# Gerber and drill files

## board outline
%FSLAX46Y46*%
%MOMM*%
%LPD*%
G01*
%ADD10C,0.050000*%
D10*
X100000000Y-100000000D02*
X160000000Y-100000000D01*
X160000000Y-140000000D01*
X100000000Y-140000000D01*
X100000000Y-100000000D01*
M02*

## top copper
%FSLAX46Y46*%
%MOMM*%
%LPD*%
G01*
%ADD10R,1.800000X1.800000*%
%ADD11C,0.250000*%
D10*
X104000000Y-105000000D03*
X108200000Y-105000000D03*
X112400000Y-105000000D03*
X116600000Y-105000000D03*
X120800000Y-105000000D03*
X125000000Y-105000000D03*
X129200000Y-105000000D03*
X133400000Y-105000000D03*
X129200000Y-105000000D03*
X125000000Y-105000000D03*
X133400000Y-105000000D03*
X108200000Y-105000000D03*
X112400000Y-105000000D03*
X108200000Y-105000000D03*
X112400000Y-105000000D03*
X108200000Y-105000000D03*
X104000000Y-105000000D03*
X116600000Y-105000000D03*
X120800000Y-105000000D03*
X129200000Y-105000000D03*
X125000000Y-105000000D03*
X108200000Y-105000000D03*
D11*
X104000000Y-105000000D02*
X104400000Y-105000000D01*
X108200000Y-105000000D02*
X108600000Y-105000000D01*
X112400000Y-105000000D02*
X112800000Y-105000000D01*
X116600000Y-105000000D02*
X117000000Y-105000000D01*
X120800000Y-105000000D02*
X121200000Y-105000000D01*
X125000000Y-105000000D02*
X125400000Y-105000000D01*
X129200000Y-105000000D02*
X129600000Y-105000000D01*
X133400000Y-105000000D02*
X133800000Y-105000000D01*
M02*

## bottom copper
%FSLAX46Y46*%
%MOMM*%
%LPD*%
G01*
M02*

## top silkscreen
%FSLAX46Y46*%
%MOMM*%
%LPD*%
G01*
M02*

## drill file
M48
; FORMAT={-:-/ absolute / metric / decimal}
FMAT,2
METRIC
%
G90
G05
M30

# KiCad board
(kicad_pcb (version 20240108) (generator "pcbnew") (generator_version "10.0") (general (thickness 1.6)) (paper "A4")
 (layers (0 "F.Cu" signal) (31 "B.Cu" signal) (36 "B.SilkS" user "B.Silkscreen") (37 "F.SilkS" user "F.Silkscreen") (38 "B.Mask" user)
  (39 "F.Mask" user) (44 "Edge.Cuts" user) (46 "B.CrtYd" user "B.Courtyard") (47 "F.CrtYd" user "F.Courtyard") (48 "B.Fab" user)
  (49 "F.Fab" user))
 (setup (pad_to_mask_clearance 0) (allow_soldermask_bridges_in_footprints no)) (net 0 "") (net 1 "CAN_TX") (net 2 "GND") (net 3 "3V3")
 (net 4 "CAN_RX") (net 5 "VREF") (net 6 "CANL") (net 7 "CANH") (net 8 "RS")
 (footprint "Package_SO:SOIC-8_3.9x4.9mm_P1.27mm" (layer "F.Cu") (at 100 100)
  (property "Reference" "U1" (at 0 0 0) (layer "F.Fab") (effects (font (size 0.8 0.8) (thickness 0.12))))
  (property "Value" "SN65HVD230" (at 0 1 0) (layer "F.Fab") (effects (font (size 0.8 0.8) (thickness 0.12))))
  (pad "1" smd rect (at 4.000 5.000) (size 1.8 1.8) (layers "F.Cu" "F.Paste" "F.Mask") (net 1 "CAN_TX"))
  (pad "2" smd rect (at 8.200 5.000) (size 1.8 1.8) (layers "F.Cu" "F.Paste" "F.Mask") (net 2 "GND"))
  (pad "3" smd rect (at 12.400 5.000) (size 1.8 1.8) (layers "F.Cu" "F.Paste" "F.Mask") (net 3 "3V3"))
  (pad "4" smd rect (at 16.600 5.000) (size 1.8 1.8) (layers "F.Cu" "F.Paste" "F.Mask") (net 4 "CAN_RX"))
  (pad "5" smd rect (at 20.800 5.000) (size 1.8 1.8) (layers "F.Cu" "F.Paste" "F.Mask") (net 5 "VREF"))
  (pad "6" smd rect (at 25.000 5.000) (size 1.8 1.8) (layers "F.Cu" "F.Paste" "F.Mask") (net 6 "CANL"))
  (pad "7" smd rect (at 29.200 5.000) (size 1.8 1.8) (layers "F.Cu" "F.Paste" "F.Mask") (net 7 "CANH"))
  (pad "8" smd rect (at 33.400 5.000) (size 1.8 1.8) (layers "F.Cu" "F.Paste" "F.Mask") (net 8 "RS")))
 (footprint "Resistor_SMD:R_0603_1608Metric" (layer "F.Cu") (at 100 100)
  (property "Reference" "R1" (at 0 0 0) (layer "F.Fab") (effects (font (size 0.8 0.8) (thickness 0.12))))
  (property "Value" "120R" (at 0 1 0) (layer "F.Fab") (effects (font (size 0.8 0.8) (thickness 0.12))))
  (pad "1" smd rect (at 29.200 5.000) (size 1.8 1.8) (layers "F.Cu" "F.Paste" "F.Mask") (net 7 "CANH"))
  (pad "2" smd rect (at 25.000 5.000) (size 1.8 1.8) (layers "F.Cu" "F.Paste" "F.Mask") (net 6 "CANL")))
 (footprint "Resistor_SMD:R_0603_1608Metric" (layer "F.Cu") (at 100 100)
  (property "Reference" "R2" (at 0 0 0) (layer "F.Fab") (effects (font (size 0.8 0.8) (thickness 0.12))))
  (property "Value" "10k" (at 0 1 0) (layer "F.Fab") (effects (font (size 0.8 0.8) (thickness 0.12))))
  (pad "1" smd rect (at 33.400 5.000) (size 1.8 1.8) (layers "F.Cu" "F.Paste" "F.Mask") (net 8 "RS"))
  (pad "2" smd rect (at 8.200 5.000) (size 1.8 1.8) (layers "F.Cu" "F.Paste" "F.Mask") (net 2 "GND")))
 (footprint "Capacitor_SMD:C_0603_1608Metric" (layer "F.Cu") (at 100 100)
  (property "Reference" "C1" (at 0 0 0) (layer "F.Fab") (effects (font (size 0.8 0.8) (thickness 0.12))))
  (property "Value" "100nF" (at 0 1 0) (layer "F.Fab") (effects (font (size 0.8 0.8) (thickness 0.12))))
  (pad "1" smd rect (at 12.400 5.000) (size 1.8 1.8) (layers "F.Cu" "F.Paste" "F.Mask") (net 3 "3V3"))
  (pad "2" smd rect (at 8.200 5.000) (size 1.8 1.8) (layers "F.Cu" "F.Paste" "F.Mask") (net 2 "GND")))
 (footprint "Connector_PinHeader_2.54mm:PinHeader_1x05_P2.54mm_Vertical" (layer "F.Cu") (at 100 100)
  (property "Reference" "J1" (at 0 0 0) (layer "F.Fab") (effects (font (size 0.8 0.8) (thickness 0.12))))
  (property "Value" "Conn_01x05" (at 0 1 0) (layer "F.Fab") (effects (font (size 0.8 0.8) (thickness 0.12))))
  (pad "1" smd rect (at 12.400 5.000) (size 1.8 1.8) (layers "F.Cu" "F.Paste" "F.Mask") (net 3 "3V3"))
  (pad "2" smd rect (at 8.200 5.000) (size 1.8 1.8) (layers "F.Cu" "F.Paste" "F.Mask") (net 2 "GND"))
  (pad "3" smd rect (at 4.000 5.000) (size 1.8 1.8) (layers "F.Cu" "F.Paste" "F.Mask") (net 1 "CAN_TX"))
  (pad "4" smd rect (at 16.600 5.000) (size 1.8 1.8) (layers "F.Cu" "F.Paste" "F.Mask") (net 4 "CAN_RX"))
  (pad "5" smd rect (at 20.800 5.000) (size 1.8 1.8) (layers "F.Cu" "F.Paste" "F.Mask") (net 5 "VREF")))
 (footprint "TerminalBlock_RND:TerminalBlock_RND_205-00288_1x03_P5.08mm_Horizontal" (layer "F.Cu") (at 100 100)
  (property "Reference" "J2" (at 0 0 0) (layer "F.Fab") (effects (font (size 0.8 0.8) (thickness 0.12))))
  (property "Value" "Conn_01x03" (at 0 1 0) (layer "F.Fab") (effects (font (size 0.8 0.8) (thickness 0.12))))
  (pad "1" smd rect (at 29.200 5.000) (size 1.8 1.8) (layers "F.Cu" "F.Paste" "F.Mask") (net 7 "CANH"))
  (pad "2" smd rect (at 25.000 5.000) (size 1.8 1.8) (layers "F.Cu" "F.Paste" "F.Mask") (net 6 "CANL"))
  (pad "3" smd rect (at 8.200 5.000) (size 1.8 1.8) (layers "F.Cu" "F.Paste" "F.Mask") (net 2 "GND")))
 (gr_rect (start 100 100) (end 160 140) (stroke (width 0.05) (type default)) (fill none) (layer "Edge.Cuts"))
 (segment (start 104.000 105.000) (end 104.400 105.000) (width 0.25) (layer "F.Cu") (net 1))
 (segment (start 108.200 105.000) (end 108.600 105.000) (width 0.25) (layer "F.Cu") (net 2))
 (segment (start 112.400 105.000) (end 112.800 105.000) (width 0.25) (layer "F.Cu") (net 3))
 (segment (start 116.600 105.000) (end 117.000 105.000) (width 0.25) (layer "F.Cu") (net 4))
 (segment (start 120.800 105.000) (end 121.200 105.000) (width 0.25) (layer "F.Cu") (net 5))
 (segment (start 125.000 105.000) (end 125.400 105.000) (width 0.25) (layer "F.Cu") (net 6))
 (segment (start 129.200 105.000) (end 129.600 105.000) (width 0.25) (layer "F.Cu") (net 7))
 (segment (start 133.400 105.000) (end 133.800 105.000) (width 0.25) (layer "F.Cu") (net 8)))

